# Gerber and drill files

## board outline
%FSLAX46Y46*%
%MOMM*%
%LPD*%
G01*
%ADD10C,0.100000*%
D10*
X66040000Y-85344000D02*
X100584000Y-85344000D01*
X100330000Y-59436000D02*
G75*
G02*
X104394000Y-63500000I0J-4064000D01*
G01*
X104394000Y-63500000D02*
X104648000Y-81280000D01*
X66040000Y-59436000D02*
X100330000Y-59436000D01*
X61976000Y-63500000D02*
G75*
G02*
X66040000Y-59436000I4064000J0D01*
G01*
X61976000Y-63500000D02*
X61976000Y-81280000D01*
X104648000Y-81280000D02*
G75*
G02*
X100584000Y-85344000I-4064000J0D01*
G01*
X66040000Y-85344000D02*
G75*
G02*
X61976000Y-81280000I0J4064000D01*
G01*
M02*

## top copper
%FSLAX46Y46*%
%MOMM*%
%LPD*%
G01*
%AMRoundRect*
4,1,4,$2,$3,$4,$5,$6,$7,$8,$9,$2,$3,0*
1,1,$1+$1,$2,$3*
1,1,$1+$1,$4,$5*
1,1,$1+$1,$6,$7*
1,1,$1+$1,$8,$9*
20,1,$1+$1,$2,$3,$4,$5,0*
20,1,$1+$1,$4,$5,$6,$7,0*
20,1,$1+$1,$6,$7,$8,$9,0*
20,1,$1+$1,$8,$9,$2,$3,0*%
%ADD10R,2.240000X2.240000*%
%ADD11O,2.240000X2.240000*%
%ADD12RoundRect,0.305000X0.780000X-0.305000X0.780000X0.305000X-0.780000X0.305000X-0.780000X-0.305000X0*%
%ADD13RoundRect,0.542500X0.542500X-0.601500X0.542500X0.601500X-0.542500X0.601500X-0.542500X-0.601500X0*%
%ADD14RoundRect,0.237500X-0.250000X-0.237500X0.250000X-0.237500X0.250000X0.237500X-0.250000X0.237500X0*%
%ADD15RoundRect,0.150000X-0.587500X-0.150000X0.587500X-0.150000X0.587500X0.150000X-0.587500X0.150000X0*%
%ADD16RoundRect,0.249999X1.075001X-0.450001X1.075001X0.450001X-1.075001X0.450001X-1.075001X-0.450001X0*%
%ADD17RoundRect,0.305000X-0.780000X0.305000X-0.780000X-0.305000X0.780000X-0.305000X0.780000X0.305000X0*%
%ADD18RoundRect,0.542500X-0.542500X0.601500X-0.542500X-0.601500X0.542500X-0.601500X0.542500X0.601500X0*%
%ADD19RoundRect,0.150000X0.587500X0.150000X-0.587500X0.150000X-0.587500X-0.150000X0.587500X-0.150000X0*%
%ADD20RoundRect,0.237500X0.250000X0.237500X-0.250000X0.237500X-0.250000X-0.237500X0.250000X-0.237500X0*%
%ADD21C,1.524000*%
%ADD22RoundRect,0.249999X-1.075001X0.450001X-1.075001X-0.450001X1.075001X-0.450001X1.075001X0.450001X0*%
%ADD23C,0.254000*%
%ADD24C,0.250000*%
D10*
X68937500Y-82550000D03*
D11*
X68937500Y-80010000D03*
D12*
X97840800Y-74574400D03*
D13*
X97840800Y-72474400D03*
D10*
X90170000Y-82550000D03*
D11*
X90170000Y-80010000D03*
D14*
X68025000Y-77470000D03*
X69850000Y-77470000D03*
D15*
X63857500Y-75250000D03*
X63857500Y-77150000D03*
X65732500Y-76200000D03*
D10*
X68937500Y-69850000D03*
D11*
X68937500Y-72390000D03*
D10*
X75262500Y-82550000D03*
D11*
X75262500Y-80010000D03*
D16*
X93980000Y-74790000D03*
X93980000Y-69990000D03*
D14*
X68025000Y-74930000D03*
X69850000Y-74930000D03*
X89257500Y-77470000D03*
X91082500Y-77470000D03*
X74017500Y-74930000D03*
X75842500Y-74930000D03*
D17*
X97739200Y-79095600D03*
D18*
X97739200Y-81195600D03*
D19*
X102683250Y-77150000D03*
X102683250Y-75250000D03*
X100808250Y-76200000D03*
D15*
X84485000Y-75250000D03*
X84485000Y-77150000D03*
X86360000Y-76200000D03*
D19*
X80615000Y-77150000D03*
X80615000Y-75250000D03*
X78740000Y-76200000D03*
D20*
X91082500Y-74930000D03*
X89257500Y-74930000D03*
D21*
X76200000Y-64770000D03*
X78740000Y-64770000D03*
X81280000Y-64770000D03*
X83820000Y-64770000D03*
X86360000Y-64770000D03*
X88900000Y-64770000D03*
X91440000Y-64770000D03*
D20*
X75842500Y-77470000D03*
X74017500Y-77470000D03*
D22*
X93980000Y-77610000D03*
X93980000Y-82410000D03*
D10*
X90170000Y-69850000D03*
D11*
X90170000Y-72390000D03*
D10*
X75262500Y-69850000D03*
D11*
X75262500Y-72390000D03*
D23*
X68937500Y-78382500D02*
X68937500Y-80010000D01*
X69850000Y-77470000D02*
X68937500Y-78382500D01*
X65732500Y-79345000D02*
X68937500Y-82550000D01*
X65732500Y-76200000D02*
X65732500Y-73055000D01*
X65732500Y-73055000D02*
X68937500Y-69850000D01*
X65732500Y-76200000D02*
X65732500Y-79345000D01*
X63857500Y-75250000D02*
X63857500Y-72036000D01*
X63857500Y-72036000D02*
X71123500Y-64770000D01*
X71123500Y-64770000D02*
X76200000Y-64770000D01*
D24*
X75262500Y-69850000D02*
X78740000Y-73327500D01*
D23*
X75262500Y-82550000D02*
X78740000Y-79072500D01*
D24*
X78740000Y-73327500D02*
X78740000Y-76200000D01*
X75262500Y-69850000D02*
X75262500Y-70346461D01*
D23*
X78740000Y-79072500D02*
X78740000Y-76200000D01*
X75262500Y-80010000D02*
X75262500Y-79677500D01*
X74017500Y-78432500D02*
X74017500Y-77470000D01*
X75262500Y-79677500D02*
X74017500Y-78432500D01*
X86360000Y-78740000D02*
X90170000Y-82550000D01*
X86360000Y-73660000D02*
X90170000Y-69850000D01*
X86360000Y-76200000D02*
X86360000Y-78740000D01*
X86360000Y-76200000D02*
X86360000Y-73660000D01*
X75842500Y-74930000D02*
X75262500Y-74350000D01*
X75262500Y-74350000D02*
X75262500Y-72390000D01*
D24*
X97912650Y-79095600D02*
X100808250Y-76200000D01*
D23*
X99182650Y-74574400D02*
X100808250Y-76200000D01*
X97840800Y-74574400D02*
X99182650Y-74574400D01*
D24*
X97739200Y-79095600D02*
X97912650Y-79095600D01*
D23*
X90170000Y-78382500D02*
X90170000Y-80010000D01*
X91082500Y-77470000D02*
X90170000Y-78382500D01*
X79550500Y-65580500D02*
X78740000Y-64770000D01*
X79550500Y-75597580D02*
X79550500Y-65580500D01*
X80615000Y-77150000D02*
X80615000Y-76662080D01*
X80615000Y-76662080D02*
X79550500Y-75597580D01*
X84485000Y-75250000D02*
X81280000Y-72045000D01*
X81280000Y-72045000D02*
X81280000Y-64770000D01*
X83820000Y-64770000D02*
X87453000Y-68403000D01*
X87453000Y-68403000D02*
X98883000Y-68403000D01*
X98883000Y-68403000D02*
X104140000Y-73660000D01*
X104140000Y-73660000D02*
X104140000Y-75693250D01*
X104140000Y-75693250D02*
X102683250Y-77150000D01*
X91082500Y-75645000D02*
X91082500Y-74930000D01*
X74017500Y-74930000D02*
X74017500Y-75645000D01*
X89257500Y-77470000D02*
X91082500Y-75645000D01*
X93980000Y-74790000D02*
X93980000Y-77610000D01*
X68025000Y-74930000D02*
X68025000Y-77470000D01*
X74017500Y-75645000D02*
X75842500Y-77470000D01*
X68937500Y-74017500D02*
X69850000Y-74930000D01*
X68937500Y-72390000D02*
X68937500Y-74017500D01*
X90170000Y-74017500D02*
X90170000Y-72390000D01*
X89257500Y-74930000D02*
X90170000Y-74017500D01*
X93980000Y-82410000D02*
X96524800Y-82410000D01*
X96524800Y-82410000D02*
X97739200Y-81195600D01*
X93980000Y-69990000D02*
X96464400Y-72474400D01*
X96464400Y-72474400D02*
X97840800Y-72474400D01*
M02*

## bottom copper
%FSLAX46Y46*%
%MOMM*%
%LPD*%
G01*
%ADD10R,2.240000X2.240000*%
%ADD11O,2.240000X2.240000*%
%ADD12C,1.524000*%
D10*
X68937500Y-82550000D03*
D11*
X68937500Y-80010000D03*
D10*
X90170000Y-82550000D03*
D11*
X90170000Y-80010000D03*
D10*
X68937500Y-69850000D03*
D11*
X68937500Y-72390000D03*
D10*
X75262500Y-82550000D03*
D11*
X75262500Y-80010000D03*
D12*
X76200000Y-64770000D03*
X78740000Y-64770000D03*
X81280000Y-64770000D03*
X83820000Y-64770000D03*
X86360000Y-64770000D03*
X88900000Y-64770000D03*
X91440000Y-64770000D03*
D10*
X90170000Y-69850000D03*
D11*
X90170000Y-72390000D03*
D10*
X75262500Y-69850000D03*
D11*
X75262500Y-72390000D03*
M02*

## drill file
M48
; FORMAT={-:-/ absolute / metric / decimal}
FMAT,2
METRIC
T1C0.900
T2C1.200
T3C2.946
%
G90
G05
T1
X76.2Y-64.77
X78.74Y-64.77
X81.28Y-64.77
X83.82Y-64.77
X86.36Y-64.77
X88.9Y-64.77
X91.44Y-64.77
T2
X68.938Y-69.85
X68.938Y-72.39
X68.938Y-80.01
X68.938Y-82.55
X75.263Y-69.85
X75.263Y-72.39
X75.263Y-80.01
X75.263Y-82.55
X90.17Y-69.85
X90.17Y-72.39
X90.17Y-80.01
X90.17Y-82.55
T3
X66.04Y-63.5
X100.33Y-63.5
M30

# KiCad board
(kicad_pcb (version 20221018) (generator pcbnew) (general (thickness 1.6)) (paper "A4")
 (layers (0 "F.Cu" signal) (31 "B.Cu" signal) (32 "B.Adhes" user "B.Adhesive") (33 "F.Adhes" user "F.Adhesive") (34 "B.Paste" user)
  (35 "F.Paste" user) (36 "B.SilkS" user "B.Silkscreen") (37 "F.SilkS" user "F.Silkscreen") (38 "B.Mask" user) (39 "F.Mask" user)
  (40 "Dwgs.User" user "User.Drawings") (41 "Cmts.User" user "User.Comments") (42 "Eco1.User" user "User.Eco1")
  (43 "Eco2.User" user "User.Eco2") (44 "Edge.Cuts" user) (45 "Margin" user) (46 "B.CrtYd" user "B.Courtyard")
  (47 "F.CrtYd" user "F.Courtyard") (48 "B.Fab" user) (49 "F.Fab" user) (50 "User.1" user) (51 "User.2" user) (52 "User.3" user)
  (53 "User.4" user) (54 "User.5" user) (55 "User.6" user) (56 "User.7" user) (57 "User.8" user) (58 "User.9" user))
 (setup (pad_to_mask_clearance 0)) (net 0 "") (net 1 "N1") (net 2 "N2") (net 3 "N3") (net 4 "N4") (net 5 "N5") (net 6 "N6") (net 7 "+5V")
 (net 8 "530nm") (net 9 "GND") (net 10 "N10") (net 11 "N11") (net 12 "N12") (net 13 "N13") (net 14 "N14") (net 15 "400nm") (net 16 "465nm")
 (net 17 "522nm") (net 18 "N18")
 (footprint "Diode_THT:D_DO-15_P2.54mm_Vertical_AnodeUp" (layer "F.Cu") (at 68.9375 82.55 90)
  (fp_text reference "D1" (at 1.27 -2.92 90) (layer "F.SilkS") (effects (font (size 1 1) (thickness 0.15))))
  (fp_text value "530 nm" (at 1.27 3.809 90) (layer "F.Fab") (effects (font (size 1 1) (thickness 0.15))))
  (pad "1" thru_hole rect (at 0 0 90) (size 2.24 2.24) (drill 1.2) (layers "*.Cu" "*.Mask") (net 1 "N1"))
  (pad "2" thru_hole oval (at 2.54 0 90) (size 2.24 2.24) (drill 1.2) (layers "*.Cu" "*.Mask") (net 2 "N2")))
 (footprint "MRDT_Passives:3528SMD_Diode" (layer "F.Cu") (at 97.79 73.66 90)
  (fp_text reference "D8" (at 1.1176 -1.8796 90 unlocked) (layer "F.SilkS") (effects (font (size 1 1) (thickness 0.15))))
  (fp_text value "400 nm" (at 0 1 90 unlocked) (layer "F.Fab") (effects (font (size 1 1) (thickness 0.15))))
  (pad "1" smd roundrect (at -0.9144 0.0508 90) (size 1.22 2.17) (layers "F.Cu" "F.Paste" "F.Mask") (roundrect_rratio 0.25) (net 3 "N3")
   (thermal_bridge_angle 45))
  (pad "2" smd roundrect (at 1.1856 0.0508 90) (size 2.288 2.17) (layers "F.Cu" "F.Paste" "F.Mask") (roundrect_rratio 0.25) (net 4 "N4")
   (thermal_bridge_angle 45)))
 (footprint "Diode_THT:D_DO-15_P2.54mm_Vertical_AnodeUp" (layer "F.Cu") (at 90.17 82.55 90)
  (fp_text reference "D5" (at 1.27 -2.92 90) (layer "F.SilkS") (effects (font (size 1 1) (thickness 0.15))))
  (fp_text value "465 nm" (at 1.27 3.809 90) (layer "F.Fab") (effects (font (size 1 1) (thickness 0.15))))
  (pad "1" thru_hole rect (at 0 0 90) (size 2.24 2.24) (drill 1.2) (layers "*.Cu" "*.Mask") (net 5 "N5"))
  (pad "2" thru_hole oval (at 2.54 0 90) (size 2.24 2.24) (drill 1.2) (layers "*.Cu" "*.Mask") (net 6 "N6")))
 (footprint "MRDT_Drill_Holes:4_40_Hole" (layer "F.Cu") (at 66.04 63.5) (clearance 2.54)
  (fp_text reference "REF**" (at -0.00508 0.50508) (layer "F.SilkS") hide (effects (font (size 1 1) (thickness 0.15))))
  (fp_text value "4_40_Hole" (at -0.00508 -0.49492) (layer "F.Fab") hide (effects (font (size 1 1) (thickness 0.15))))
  (pad "" np_thru_hole circle (at 0 0) (size 2.9464 2.9464) (drill 2.9464) (layers "*.Cu" "*.Mask") (clearance 2.5)))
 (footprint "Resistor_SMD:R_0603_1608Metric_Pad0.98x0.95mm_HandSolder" (layer "F.Cu") (at 68.9375 77.47)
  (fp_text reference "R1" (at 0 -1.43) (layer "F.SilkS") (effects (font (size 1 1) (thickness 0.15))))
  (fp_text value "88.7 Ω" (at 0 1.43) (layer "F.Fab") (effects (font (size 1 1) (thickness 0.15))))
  (pad "1" smd roundrect (at -0.9125 0) (size 0.975 0.95) (layers "F.Cu" "F.Paste" "F.Mask") (roundrect_rratio 0.25) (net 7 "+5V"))
  (pad "2" smd roundrect (at 0.9125 0) (size 0.975 0.95) (layers "F.Cu" "F.Paste" "F.Mask") (roundrect_rratio 0.25) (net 2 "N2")))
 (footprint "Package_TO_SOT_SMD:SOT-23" (layer "F.Cu") (at 64.795 76.2)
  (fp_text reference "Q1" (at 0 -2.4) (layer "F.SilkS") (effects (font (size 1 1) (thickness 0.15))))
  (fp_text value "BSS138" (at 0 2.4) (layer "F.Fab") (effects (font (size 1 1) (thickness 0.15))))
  (pad "1" smd roundrect (at -0.9375 -0.95) (size 1.475 0.6) (layers "F.Cu" "F.Paste" "F.Mask") (roundrect_rratio 0.25) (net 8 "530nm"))
  (pad "2" smd roundrect (at -0.9375 0.95) (size 1.475 0.6) (layers "F.Cu" "F.Paste" "F.Mask") (roundrect_rratio 0.25) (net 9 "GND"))
  (pad "3" smd roundrect (at 0.9375 0) (size 1.475 0.6) (layers "F.Cu" "F.Paste" "F.Mask") (roundrect_rratio 0.25) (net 1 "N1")))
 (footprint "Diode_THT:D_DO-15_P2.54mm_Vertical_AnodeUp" (layer "F.Cu") (at 68.9375 69.85 -90)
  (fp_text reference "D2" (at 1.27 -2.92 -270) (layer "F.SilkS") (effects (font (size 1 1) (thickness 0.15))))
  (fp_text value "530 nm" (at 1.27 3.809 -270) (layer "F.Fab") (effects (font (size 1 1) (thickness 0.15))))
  (pad "1" thru_hole rect (at 0 0 270) (size 2.24 2.24) (drill 1.2) (layers "*.Cu" "*.Mask") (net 1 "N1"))
  (pad "2" thru_hole oval (at 2.54 0 270) (size 2.24 2.24) (drill 1.2) (layers "*.Cu" "*.Mask") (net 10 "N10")))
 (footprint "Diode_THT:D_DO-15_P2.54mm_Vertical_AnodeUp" (layer "F.Cu") (at 75.2625 82.55 90)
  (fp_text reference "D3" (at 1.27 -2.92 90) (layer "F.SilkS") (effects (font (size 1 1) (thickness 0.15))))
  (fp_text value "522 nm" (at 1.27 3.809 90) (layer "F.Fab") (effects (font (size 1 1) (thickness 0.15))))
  (pad "1" thru_hole rect (at 0 0 90) (size 2.24 2.24) (drill 1.2) (layers "*.Cu" "*.Mask") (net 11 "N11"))
  (pad "2" thru_hole oval (at 2.54 0 90) (size 2.24 2.24) (drill 1.2) (layers "*.Cu" "*.Mask") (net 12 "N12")))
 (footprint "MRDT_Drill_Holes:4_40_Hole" (layer "F.Cu") (at 100.33 63.5) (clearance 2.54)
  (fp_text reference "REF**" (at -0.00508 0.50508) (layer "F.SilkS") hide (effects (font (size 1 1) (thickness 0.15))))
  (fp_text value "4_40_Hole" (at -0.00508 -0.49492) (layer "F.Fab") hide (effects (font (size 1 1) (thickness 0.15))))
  (pad "" np_thru_hole circle (at 0 0) (size 2.9464 2.9464) (drill 2.9464) (layers "F&B.Cu" "*.Mask") (clearance 2.5)))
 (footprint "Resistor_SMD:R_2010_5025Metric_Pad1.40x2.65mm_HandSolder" (layer "F.Cu") (at 93.98 72.39 90)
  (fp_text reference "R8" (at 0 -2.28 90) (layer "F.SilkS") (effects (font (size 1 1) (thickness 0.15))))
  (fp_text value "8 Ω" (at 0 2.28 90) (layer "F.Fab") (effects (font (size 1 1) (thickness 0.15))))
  (pad "1" smd roundrect (at -2.4 0 90) (size 1.4 2.65) (layers "F.Cu" "F.Paste" "F.Mask") (roundrect_rratio 0.178571) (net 7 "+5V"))
  (pad "2" smd roundrect (at 2.4 0 90) (size 1.4 2.65) (layers "F.Cu" "F.Paste" "F.Mask") (roundrect_rratio 0.178571) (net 4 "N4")))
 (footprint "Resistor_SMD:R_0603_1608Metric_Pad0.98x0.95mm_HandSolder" (layer "F.Cu") (at 68.9375 74.93)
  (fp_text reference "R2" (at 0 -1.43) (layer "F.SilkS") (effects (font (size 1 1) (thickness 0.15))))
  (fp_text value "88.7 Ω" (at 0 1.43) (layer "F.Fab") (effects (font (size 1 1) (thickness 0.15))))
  (pad "1" smd roundrect (at -0.9125 0) (size 0.975 0.95) (layers "F.Cu" "F.Paste" "F.Mask") (roundrect_rratio 0.25) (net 7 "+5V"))
  (pad "2" smd roundrect (at 0.9125 0) (size 0.975 0.95) (layers "F.Cu" "F.Paste" "F.Mask") (roundrect_rratio 0.25) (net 10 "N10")))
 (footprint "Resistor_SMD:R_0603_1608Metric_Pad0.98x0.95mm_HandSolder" (layer "F.Cu") (at 90.17 77.47)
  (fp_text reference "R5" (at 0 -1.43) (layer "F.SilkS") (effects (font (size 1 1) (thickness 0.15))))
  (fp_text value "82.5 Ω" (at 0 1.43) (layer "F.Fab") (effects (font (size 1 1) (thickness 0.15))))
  (pad "1" smd roundrect (at -0.9125 0) (size 0.975 0.95) (layers "F.Cu" "F.Paste" "F.Mask") (roundrect_rratio 0.25) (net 7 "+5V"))
  (pad "2" smd roundrect (at 0.9125 0) (size 0.975 0.95) (layers "F.Cu" "F.Paste" "F.Mask") (roundrect_rratio 0.25) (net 6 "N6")))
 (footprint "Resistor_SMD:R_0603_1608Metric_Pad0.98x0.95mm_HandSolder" (layer "F.Cu") (at 74.93 74.93)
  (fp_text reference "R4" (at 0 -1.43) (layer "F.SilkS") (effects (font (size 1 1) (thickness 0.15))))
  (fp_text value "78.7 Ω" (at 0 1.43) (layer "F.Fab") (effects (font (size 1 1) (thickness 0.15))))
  (pad "1" smd roundrect (at -0.9125 0) (size 0.975 0.95) (layers "F.Cu" "F.Paste" "F.Mask") (roundrect_rratio 0.25) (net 7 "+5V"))
  (pad "2" smd roundrect (at 0.9125 0) (size 0.975 0.95) (layers "F.Cu" "F.Paste" "F.Mask") (roundrect_rratio 0.25) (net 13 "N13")))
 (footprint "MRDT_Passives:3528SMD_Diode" (layer "F.Cu") (at 97.79 80.01 -90)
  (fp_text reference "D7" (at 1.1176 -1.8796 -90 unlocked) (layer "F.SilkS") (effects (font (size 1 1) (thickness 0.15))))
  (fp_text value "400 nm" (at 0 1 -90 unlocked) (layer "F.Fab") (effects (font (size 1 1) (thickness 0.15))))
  (pad "1" smd roundrect (at -0.9144 0.0508 270) (size 1.22 2.17) (layers "F.Cu" "F.Paste" "F.Mask") (roundrect_rratio 0.25) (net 3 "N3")
   (thermal_bridge_angle 45))
  (pad "2" smd roundrect (at 1.1856 0.0508 270) (size 2.288 2.17) (layers "F.Cu" "F.Paste" "F.Mask") (roundrect_rratio 0.25) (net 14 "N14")
   (thermal_bridge_angle 45)))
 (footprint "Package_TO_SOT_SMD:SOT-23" (layer "F.Cu") (at 101.74575 76.2 180)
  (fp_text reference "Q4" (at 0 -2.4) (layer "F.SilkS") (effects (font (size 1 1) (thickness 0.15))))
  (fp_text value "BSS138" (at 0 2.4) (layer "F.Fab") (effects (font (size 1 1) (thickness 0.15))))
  (pad "1" smd roundrect (at -0.9375 -0.95 180) (size 1.475 0.6) (layers "F.Cu" "F.Paste" "F.Mask") (roundrect_rratio 0.25) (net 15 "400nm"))
  (pad "2" smd roundrect (at -0.9375 0.95 180) (size 1.475 0.6) (layers "F.Cu" "F.Paste" "F.Mask") (roundrect_rratio 0.25) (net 9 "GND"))
  (pad "3" smd roundrect (at 0.9375 0 180) (size 1.475 0.6) (layers "F.Cu" "F.Paste" "F.Mask") (roundrect_rratio 0.25) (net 3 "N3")))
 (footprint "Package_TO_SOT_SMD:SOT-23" (layer "F.Cu") (at 85.4225 76.2)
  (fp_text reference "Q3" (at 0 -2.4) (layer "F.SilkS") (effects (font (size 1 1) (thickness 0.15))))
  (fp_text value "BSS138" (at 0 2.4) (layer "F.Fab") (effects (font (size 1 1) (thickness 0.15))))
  (pad "1" smd roundrect (at -0.9375 -0.95) (size 1.475 0.6) (layers "F.Cu" "F.Paste" "F.Mask") (roundrect_rratio 0.25) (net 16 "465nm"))
  (pad "2" smd roundrect (at -0.9375 0.95) (size 1.475 0.6) (layers "F.Cu" "F.Paste" "F.Mask") (roundrect_rratio 0.25) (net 9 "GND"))
  (pad "3" smd roundrect (at 0.9375 0) (size 1.475 0.6) (layers "F.Cu" "F.Paste" "F.Mask") (roundrect_rratio 0.25) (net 5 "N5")))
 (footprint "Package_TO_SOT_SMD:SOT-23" (layer "F.Cu") (at 79.6775 76.2 180)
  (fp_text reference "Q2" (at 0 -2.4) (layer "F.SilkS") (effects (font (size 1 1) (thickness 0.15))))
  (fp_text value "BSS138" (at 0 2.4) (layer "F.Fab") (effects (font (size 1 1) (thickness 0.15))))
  (pad "1" smd roundrect (at -0.9375 -0.95 180) (size 1.475 0.6) (layers "F.Cu" "F.Paste" "F.Mask") (roundrect_rratio 0.25) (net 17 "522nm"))
  (pad "2" smd roundrect (at -0.9375 0.95 180) (size 1.475 0.6) (layers "F.Cu" "F.Paste" "F.Mask") (roundrect_rratio 0.25) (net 9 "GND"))
  (pad "3" smd roundrect (at 0.9375 0 180) (size 1.475 0.6) (layers "F.Cu" "F.Paste" "F.Mask") (roundrect_rratio 0.25) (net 11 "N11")))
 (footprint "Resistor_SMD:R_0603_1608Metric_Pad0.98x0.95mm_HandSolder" (layer "F.Cu") (at 90.17 74.93 180)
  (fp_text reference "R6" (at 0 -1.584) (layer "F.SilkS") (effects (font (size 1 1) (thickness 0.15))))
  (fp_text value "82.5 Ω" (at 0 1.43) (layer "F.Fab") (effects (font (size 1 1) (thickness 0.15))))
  (pad "1" smd roundrect (at -0.9125 0 180) (size 0.975 0.95) (layers "F.Cu" "F.Paste" "F.Mask") (roundrect_rratio 0.25) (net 7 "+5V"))
  (pad "2" smd roundrect (at 0.9125 0 180) (size 0.975 0.95) (layers "F.Cu" "F.Paste" "F.Mask") (roundrect_rratio 0.25) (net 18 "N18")))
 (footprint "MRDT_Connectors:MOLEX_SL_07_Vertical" (layer "F.Cu") (at 76.2 64.77)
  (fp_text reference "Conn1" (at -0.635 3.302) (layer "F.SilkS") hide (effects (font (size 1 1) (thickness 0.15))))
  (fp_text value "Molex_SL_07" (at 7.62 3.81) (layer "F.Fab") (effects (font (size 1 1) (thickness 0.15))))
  (pad "1" thru_hole circle (at 0 0) (size 1.524 1.524) (drill 0.9) (layers "*.Cu" "*.Mask") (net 8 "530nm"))
  (pad "2" thru_hole circle (at 2.54 0) (size 1.524 1.524) (drill 0.9) (layers "*.Cu" "*.Mask") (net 17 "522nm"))
  (pad "3" thru_hole circle (at 5.08 0) (size 1.524 1.524) (drill 0.9) (layers "*.Cu" "*.Mask") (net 16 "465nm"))
  (pad "4" thru_hole circle (at 7.62 0) (size 1.524 1.524) (drill 0.9) (layers "*.Cu" "*.Mask") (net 15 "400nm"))
  (pad "5" thru_hole circle (at 10.16 0) (size 1.524 1.524) (drill 0.9) (layers "*.Cu" "*.Mask") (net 7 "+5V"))
  (pad "6" thru_hole circle (at 12.7 0) (size 1.524 1.524) (drill 0.9) (layers "*.Cu" "*.Mask") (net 9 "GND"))
  (pad "7" thru_hole circle (at 15.24 0) (size 1.524 1.524) (drill 0.9) (layers "*.Cu" "*.Mask") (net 9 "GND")))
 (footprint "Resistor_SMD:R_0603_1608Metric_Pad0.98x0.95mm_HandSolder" (layer "F.Cu") (at 74.93 77.47 180)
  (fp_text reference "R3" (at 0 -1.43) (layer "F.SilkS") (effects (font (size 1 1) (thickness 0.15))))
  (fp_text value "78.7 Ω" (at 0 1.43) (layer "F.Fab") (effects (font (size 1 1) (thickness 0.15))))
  (pad "1" smd roundrect (at -0.9125 0 180) (size 0.975 0.95) (layers "F.Cu" "F.Paste" "F.Mask") (roundrect_rratio 0.25) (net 7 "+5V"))
  (pad "2" smd roundrect (at 0.9125 0 180) (size 0.975 0.95) (layers "F.Cu" "F.Paste" "F.Mask") (roundrect_rratio 0.25) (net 12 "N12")))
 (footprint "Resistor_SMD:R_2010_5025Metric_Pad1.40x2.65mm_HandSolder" (layer "F.Cu") (at 93.98 80.01 -90)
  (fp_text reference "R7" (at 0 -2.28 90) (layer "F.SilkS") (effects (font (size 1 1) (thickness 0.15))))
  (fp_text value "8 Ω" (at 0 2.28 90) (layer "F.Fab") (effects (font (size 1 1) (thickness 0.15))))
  (pad "1" smd roundrect (at -2.4 0 270) (size 1.4 2.65) (layers "F.Cu" "F.Paste" "F.Mask") (roundrect_rratio 0.178571) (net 7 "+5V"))
  (pad "2" smd roundrect (at 2.4 0 270) (size 1.4 2.65) (layers "F.Cu" "F.Paste" "F.Mask") (roundrect_rratio 0.178571) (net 14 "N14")))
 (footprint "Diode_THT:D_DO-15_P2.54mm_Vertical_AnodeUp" (layer "F.Cu") (at 90.17 69.85 -90)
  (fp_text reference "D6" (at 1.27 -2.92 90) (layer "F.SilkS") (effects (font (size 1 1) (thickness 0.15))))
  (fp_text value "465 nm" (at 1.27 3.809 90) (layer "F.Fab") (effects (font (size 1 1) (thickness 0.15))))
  (pad "1" thru_hole rect (at 0 0 270) (size 2.24 2.24) (drill 1.2) (layers "*.Cu" "*.Mask") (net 5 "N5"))
  (pad "2" thru_hole oval (at 2.54 0 270) (size 2.24 2.24) (drill 1.2) (layers "*.Cu" "*.Mask") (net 18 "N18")))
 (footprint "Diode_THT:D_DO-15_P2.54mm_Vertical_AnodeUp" (layer "F.Cu") (at 75.2625 69.85 -90)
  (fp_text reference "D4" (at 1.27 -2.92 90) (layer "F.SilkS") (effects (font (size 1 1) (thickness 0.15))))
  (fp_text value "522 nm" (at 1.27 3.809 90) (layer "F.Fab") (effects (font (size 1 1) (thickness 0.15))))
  (pad "1" thru_hole rect (at 0 0 270) (size 2.24 2.24) (drill 1.2) (layers "*.Cu" "*.Mask") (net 11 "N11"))
  (pad "2" thru_hole oval (at 2.54 0 270) (size 2.24 2.24) (drill 1.2) (layers "*.Cu" "*.Mask") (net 13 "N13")))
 (gr_line (start 66.04 85.344) (end 100.584 85.344) (stroke (width 0.1) (type default)) (layer "Edge.Cuts"))
 (gr_arc (start 100.33 59.436) (mid 103.203682 60.626318) (end 104.394 63.5) (stroke (width 0.1) (type default)) (layer "Edge.Cuts"))
 (gr_line (start 104.394 63.5) (end 104.648 81.28) (stroke (width 0.1) (type default)) (layer "Edge.Cuts"))
 (gr_line (start 66.04 59.436) (end 100.33 59.436) (stroke (width 0.1) (type default)) (layer "Edge.Cuts"))
 (gr_arc (start 61.976 63.5) (mid 63.166318 60.626318) (end 66.04 59.436) (stroke (width 0.1) (type default)) (layer "Edge.Cuts"))
 (gr_line (start 61.976 63.5) (end 61.976 81.28) (stroke (width 0.1) (type default)) (layer "Edge.Cuts"))
 (gr_arc (start 104.648 81.28) (mid 103.457682 84.153682) (end 100.584 85.344) (stroke (width 0.1) (type default)) (layer "Edge.Cuts"))
 (gr_arc (start 66.04 85.344) (mid 63.166318 84.153682) (end 61.976 81.28) (stroke (width 0.1) (type default)) (layer "Edge.Cuts"))
 (segment (start 68.9375 78.3825) (end 68.9375 80.01) (width 0.254) (layer "F.Cu") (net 2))
 (segment (start 69.85 77.47) (end 68.9375 78.3825) (width 0.254) (layer "F.Cu") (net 2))
 (segment (start 65.7325 79.345) (end 68.9375 82.55) (width 0.254) (layer "F.Cu") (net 1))
 (segment (start 65.7325 76.2) (end 65.7325 73.055) (width 0.254) (layer "F.Cu") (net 1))
 (segment (start 65.7325 73.055) (end 68.9375 69.85) (width 0.254) (layer "F.Cu") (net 1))
 (segment (start 65.7325 76.2) (end 65.7325 79.345) (width 0.254) (layer "F.Cu") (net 1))
 (segment (start 63.8575 75.25) (end 63.8575 72.036) (width 0.254) (layer "F.Cu") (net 8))
 (segment (start 63.8575 72.036) (end 71.1235 64.77) (width 0.254) (layer "F.Cu") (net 8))
 (segment (start 71.1235 64.77) (end 76.2 64.77) (width 0.254) (layer "F.Cu") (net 8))
 (segment (start 75.2625 69.85) (end 78.74 73.3275) (width 0.25) (layer "F.Cu") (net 11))
 (segment (start 75.2625 82.55) (end 78.74 79.0725) (width 0.254) (layer "F.Cu") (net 11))
 (segment (start 78.74 73.3275) (end 78.74 76.2) (width 0.25) (layer "F.Cu") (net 11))
 (segment (start 75.2625 69.85) (end 75.2625 70.346461) (width 0.25) (layer "F.Cu") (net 11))
 (segment (start 78.74 79.0725) (end 78.74 76.2) (width 0.254) (layer "F.Cu") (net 11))
 (segment (start 75.2625 80.01) (end 75.2625 79.6775) (width 0.254) (layer "F.Cu") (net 12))
 (segment (start 74.0175 78.4325) (end 74.0175 77.47) (width 0.254) (layer "F.Cu") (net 12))
 (segment (start 75.2625 79.6775) (end 74.0175 78.4325) (width 0.254) (layer "F.Cu") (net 12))
 (segment (start 86.36 78.74) (end 90.17 82.55) (width 0.254) (layer "F.Cu") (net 5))
 (segment (start 86.36 73.66) (end 90.17 69.85) (width 0.254) (layer "F.Cu") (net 5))
 (segment (start 86.36 76.2) (end 86.36 78.74) (width 0.254) (layer "F.Cu") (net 5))
 (segment (start 86.36 76.2) (end 86.36 73.66) (width 0.254) (layer "F.Cu") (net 5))
 (segment (start 75.8425 74.93) (end 75.2625 74.35) (width 0.254) (layer "F.Cu") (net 13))
 (segment (start 75.2625 74.35) (end 75.2625 72.39) (width 0.254) (layer "F.Cu") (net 13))
 (segment (start 97.91265 79.0956) (end 100.80825 76.2) (width 0.25) (layer "F.Cu") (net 3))
 (segment (start 99.18265 74.5744) (end 100.80825 76.2) (width 0.254) (layer "F.Cu") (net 3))
 (segment (start 97.8408 74.5744) (end 99.18265 74.5744) (width 0.254) (layer "F.Cu") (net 3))
 (segment (start 97.7392 79.0956) (end 97.91265 79.0956) (width 0.25) (layer "F.Cu") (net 3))
 (segment (start 90.17 78.3825) (end 90.17 80.01) (width 0.254) (layer "F.Cu") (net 6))
 (segment (start 91.0825 77.47) (end 90.17 78.3825) (width 0.254) (layer "F.Cu") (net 6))
 (segment (start 79.5505 65.5805) (end 78.74 64.77) (width 0.254) (layer "F.Cu") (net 17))
 (segment (start 79.5505 75.59758) (end 79.5505 65.5805) (width 0.254) (layer "F.Cu") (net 17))
 (segment (start 80.615 77.15) (end 80.615 76.66208) (width 0.254) (layer "F.Cu") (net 17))
 (segment (start 80.615 76.66208) (end 79.5505 75.59758) (width 0.254) (layer "F.Cu") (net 17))
 (segment (start 84.485 75.25) (end 81.28 72.045) (width 0.254) (layer "F.Cu") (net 16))
 (segment (start 81.28 72.045) (end 81.28 64.77) (width 0.254) (layer "F.Cu") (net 16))
 (segment (start 83.82 64.77) (end 87.453 68.403) (width 0.254) (layer "F.Cu") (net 15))
 (segment (start 87.453 68.403) (end 98.883 68.403) (width 0.254) (layer "F.Cu") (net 15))
 (segment (start 98.883 68.403) (end 104.14 73.66) (width 0.254) (layer "F.Cu") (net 15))
 (segment (start 104.14 73.66) (end 104.14 75.69325) (width 0.254) (layer "F.Cu") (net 15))
 (segment (start 104.14 75.69325) (end 102.68325 77.15) (width 0.254) (layer "F.Cu") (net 15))
 (segment (start 91.0825 75.645) (end 91.0825 74.93) (width 0.254) (layer "F.Cu") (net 7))
 (segment (start 74.0175 74.93) (end 74.0175 75.645) (width 0.254) (layer "F.Cu") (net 7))
 (segment (start 89.2575 77.47) (end 91.0825 75.645) (width 0.254) (layer "F.Cu") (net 7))
 (segment (start 93.98 74.79) (end 93.98 77.61) (width 0.254) (layer "F.Cu") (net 7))
 (segment (start 68.025 74.93) (end 68.025 77.47) (width 0.254) (layer "F.Cu") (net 7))
 (segment (start 74.0175 75.645) (end 75.8425 77.47) (width 0.254) (layer "F.Cu") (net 7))
 (segment (start 68.9375 74.0175) (end 69.85 74.93) (width 0.254) (layer "F.Cu") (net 10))
 (segment (start 68.9375 72.39) (end 68.9375 74.0175) (width 0.254) (layer "F.Cu") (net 10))
 (segment (start 90.17 74.0175) (end 90.17 72.39) (width 0.254) (layer "F.Cu") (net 18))
 (segment (start 89.2575 74.93) (end 90.17 74.0175) (width 0.254) (layer "F.Cu") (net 18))
 (segment (start 93.98 82.41) (end 96.5248 82.41) (width 0.254) (layer "F.Cu") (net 14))
 (segment (start 96.5248 82.41) (end 97.7392 81.1956) (width 0.254) (layer "F.Cu") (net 14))
 (segment (start 93.98 69.99) (end 96.4644 72.4744) (width 0.254) (layer "F.Cu") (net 4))
 (segment (start 96.4644 72.4744) (end 97.8408 72.4744) (width 0.254) (layer "F.Cu") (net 4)))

